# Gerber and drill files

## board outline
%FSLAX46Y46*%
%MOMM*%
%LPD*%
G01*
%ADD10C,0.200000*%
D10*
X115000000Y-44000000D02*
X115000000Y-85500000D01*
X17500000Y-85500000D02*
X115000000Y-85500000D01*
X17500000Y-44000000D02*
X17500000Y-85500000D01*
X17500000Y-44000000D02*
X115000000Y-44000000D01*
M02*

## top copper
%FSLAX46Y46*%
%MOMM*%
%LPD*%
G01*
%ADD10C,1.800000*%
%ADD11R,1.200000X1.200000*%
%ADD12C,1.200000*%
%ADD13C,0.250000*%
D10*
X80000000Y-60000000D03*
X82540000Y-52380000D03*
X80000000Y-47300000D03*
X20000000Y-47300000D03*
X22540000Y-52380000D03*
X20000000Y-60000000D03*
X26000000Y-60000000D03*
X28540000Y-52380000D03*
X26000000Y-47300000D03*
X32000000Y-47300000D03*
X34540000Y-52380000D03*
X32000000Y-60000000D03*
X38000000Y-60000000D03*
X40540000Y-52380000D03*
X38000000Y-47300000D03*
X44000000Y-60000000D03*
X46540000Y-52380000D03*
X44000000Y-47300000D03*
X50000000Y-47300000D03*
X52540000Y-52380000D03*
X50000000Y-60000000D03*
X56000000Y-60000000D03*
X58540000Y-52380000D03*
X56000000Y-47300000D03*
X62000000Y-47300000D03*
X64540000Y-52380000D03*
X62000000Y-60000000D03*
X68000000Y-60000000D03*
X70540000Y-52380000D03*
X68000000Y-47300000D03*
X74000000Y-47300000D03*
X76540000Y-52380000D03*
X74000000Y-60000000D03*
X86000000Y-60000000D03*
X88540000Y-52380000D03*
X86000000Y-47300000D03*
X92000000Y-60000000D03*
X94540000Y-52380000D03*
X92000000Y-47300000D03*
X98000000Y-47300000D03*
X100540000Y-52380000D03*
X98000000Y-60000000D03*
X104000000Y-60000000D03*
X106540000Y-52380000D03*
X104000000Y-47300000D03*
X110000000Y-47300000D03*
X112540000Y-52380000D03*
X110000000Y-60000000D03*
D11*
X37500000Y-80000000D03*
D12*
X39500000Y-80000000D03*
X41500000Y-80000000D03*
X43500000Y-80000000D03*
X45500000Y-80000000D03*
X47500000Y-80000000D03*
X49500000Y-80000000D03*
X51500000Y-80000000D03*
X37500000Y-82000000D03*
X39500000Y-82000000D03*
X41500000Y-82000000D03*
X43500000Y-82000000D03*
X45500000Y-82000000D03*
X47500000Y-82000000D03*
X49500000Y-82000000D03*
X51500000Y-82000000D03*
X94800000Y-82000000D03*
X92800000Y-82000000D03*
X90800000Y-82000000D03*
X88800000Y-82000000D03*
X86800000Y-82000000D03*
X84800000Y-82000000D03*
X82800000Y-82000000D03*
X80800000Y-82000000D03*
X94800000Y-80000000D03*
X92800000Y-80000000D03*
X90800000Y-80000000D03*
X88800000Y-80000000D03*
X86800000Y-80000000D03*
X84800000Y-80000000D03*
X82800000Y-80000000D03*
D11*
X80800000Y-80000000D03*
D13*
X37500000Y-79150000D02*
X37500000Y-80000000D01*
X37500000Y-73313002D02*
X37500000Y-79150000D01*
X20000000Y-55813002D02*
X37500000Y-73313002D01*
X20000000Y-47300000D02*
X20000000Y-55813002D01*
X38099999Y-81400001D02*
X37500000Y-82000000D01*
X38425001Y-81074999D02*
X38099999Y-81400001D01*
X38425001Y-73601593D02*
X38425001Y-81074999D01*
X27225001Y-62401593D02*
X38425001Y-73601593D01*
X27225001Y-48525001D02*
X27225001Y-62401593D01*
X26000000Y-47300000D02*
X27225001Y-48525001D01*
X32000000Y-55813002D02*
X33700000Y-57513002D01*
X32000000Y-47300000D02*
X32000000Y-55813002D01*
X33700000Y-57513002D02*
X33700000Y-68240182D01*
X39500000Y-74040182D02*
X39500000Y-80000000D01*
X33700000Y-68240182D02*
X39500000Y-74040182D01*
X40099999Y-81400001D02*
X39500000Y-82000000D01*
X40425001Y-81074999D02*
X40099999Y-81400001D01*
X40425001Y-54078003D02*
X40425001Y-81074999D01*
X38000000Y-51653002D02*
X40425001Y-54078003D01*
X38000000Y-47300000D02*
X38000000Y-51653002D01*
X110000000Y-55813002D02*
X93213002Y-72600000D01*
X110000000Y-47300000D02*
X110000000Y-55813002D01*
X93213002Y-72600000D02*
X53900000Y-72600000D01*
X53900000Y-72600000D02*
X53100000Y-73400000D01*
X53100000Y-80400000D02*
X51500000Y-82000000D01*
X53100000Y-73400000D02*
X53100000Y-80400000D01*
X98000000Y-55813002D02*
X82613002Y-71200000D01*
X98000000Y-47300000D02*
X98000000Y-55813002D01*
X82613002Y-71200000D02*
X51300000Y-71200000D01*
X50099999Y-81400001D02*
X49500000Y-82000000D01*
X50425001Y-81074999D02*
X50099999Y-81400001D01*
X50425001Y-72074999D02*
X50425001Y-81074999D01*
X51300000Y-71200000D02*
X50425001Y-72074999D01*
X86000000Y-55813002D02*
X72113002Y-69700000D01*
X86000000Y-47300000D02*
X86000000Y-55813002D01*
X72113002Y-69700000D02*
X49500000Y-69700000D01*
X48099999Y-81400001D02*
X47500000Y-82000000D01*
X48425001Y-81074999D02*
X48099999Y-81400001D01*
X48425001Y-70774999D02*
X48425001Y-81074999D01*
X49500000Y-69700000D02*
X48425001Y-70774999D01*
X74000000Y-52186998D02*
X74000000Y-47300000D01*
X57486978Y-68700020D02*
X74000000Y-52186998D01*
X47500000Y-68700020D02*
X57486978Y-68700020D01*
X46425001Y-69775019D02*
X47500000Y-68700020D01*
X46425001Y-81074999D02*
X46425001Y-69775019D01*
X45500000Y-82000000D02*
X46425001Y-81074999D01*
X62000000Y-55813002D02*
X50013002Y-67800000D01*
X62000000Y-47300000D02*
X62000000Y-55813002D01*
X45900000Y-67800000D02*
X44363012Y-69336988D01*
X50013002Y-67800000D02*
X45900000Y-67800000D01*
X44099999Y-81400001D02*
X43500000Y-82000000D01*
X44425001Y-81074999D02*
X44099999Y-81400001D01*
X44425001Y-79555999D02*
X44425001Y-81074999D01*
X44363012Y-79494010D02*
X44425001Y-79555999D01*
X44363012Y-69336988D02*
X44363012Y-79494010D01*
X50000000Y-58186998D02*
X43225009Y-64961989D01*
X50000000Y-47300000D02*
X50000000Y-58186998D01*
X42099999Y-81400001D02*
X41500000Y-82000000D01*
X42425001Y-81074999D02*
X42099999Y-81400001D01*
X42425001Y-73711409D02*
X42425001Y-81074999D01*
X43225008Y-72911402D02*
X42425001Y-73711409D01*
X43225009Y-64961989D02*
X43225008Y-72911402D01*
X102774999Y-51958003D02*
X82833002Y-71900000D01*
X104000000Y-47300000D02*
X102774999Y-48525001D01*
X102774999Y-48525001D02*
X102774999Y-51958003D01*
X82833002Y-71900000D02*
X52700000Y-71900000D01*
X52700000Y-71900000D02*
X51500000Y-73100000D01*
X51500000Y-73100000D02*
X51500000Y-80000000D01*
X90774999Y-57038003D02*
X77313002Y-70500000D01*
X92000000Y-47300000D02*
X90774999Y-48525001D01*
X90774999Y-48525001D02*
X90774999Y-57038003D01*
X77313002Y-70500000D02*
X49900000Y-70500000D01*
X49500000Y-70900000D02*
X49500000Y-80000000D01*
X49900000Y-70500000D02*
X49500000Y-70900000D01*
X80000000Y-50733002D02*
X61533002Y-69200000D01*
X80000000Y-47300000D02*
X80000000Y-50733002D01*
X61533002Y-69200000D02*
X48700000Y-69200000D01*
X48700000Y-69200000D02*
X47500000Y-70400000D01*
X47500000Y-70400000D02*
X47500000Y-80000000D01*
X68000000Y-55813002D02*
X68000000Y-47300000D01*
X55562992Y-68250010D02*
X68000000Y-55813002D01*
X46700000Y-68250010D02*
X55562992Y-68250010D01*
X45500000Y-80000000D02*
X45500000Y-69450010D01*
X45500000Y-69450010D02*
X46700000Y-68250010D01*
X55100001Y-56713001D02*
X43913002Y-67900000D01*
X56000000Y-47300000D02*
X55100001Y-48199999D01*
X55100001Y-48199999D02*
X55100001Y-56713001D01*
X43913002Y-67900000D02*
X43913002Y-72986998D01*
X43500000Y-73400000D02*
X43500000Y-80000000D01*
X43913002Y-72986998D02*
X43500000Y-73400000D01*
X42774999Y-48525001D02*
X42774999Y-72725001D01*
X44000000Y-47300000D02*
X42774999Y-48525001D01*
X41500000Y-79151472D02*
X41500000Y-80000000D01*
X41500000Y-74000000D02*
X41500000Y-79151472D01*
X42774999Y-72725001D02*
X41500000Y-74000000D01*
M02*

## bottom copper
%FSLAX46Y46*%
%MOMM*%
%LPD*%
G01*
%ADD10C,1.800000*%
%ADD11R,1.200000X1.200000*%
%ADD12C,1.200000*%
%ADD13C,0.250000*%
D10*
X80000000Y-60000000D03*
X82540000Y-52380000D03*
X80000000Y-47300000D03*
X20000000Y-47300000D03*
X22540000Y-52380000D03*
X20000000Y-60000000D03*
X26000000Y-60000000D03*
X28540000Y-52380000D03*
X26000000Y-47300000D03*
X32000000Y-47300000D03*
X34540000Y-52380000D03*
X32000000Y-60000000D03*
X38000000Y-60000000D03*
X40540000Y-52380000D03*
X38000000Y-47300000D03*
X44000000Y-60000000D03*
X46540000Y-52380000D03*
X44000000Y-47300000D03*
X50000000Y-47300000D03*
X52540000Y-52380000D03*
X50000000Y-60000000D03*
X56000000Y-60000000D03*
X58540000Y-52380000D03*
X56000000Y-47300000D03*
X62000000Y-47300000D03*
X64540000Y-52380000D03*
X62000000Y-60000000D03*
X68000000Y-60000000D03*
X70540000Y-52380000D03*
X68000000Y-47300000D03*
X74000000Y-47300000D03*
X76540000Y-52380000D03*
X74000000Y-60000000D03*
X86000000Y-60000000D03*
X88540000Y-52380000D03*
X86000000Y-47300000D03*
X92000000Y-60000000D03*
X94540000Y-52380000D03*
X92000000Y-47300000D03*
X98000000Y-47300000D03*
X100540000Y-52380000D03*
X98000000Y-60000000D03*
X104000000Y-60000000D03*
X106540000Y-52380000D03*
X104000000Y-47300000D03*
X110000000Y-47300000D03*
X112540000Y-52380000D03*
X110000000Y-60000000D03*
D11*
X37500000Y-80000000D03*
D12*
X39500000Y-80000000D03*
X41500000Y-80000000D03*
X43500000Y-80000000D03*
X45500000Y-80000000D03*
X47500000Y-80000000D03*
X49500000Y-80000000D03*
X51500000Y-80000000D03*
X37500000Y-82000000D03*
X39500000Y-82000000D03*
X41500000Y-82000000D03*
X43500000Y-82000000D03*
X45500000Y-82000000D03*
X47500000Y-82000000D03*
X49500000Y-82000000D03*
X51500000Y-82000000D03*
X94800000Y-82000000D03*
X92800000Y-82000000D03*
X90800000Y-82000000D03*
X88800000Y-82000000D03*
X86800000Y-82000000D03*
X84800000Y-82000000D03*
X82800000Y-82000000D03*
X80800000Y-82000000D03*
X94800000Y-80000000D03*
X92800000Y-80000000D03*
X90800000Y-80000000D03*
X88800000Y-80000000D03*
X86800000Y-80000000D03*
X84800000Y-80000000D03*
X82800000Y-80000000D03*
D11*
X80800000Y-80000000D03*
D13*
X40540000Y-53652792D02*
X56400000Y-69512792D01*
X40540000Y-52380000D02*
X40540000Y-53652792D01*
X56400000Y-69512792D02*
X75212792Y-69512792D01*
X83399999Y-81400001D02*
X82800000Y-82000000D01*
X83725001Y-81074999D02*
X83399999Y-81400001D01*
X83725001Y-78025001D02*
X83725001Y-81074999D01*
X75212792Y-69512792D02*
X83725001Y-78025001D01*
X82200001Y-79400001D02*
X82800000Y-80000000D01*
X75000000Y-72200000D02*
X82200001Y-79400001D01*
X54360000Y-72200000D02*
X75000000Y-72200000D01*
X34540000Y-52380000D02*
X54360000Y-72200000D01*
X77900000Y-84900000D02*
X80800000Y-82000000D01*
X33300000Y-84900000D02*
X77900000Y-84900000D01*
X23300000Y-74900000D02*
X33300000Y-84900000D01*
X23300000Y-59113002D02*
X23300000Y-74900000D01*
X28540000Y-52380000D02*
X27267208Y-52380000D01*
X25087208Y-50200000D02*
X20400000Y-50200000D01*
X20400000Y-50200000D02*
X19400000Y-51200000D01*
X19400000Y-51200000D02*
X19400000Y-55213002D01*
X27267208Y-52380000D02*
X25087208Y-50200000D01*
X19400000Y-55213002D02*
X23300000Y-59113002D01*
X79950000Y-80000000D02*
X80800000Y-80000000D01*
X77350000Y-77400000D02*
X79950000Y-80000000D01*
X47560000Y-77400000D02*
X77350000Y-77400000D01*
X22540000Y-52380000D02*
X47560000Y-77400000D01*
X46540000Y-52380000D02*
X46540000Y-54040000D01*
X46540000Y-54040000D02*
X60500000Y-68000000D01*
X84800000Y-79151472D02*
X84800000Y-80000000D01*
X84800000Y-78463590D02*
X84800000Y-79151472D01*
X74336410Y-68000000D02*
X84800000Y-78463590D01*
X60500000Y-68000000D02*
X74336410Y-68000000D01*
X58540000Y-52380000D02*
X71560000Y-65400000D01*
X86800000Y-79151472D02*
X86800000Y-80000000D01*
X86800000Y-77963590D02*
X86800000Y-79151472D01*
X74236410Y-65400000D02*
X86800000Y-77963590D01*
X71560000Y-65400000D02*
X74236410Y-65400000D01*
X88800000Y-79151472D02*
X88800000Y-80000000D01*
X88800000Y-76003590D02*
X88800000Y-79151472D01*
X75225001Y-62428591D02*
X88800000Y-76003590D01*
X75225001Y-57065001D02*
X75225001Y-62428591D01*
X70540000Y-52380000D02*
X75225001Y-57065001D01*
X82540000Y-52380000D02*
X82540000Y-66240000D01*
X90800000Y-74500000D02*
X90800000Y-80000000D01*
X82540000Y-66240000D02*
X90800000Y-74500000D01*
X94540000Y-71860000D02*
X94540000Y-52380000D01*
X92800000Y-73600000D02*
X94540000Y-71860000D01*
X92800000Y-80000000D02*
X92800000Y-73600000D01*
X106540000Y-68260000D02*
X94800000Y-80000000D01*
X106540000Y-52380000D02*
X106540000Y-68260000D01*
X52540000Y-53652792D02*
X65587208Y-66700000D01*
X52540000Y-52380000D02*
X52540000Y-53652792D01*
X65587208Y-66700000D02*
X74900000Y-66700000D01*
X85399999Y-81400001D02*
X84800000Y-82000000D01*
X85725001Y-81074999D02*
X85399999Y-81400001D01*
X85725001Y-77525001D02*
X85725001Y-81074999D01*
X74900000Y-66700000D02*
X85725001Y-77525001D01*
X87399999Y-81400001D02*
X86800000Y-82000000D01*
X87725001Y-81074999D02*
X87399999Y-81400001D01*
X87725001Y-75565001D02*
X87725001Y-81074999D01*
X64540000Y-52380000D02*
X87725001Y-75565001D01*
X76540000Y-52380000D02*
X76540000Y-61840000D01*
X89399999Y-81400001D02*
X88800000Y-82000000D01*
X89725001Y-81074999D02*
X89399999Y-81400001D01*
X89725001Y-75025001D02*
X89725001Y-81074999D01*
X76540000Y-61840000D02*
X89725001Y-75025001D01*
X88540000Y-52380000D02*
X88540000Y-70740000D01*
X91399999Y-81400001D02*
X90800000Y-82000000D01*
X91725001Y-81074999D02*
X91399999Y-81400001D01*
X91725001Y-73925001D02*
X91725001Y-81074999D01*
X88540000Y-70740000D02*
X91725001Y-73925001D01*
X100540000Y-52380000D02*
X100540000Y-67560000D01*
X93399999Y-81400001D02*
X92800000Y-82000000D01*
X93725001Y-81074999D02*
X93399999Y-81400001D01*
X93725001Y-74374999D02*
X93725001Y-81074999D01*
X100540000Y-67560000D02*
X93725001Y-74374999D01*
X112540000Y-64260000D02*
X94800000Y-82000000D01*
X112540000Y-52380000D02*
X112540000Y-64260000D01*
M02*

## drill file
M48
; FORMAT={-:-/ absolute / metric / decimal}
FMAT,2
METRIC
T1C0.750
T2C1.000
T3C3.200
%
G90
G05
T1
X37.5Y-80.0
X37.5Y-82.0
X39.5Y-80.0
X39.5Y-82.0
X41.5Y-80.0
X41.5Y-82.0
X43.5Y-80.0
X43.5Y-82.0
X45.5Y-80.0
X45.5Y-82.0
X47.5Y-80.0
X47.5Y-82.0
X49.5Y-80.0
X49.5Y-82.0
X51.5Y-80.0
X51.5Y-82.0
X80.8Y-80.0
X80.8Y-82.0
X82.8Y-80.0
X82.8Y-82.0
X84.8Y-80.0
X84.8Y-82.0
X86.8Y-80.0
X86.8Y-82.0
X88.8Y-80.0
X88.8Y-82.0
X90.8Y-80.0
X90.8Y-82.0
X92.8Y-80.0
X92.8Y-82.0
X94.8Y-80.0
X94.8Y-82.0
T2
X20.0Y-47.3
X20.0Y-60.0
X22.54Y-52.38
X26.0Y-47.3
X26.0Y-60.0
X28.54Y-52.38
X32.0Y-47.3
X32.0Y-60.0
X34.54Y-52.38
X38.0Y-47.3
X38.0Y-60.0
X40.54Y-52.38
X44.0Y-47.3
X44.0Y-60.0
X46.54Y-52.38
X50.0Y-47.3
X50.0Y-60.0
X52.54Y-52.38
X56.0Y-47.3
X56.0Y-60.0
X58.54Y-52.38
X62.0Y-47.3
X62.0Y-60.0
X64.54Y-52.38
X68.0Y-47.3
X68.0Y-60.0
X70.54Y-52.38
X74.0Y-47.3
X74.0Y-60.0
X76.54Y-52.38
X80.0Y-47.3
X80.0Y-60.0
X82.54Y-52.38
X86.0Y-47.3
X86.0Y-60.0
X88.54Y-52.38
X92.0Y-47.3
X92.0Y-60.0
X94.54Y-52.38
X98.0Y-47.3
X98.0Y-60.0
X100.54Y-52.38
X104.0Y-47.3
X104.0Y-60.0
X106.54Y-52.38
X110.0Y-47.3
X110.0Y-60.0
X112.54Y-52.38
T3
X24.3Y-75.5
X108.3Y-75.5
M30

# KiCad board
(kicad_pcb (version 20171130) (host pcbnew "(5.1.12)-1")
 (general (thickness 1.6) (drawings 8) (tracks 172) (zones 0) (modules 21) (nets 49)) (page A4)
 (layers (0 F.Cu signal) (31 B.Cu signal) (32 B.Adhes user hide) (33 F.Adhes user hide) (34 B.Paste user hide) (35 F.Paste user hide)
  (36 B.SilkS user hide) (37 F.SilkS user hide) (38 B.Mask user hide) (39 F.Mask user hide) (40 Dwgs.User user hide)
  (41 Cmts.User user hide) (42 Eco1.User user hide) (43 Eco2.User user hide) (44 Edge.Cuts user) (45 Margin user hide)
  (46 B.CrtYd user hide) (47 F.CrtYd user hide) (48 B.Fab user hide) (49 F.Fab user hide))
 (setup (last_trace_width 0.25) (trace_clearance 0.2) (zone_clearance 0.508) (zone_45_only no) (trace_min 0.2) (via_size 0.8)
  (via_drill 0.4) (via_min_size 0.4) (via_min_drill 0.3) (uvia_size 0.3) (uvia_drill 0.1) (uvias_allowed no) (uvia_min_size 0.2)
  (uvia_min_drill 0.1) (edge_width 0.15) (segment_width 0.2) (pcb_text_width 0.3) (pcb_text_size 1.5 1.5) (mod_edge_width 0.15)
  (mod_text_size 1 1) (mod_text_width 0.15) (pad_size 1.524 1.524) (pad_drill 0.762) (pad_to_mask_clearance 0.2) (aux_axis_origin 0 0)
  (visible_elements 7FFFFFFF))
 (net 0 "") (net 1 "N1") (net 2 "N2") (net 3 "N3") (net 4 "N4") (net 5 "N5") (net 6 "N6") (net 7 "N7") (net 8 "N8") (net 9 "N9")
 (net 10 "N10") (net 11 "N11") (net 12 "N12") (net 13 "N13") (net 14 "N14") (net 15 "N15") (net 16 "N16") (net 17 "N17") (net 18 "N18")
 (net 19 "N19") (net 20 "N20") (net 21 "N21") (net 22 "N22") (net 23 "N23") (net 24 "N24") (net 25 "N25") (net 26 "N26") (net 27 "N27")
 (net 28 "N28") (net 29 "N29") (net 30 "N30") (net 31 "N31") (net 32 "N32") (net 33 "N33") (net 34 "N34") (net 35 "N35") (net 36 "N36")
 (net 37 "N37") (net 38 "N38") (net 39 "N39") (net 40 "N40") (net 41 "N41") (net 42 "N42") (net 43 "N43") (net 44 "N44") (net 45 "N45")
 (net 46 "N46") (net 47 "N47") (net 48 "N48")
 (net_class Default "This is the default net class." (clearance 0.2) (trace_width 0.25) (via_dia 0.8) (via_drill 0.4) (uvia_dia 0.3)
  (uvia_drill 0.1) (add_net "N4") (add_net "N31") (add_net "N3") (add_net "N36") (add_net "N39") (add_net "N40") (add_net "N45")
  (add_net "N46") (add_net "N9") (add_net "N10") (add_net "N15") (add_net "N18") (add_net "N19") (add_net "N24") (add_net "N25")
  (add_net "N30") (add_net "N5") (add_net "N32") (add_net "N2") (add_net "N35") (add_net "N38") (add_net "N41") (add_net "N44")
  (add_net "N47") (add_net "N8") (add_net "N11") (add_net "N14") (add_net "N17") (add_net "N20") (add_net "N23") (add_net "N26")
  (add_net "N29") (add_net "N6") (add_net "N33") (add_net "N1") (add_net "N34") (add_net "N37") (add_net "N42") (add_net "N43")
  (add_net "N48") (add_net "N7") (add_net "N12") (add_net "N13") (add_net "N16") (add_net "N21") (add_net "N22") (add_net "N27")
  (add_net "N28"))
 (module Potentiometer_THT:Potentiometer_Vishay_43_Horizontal (layer F.Cu) (at 80 60 270)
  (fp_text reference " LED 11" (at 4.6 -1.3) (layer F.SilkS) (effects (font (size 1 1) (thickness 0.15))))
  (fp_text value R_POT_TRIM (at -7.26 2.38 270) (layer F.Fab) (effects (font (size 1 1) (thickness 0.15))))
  (pad 1 thru_hole circle (at 0 0 270) (size 1.8 1.8) (drill 1) (layers *.Cu *.Mask) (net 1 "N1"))
  (pad 2 thru_hole circle (at -7.62 -2.54 270) (size 1.8 1.8) (drill 1) (layers *.Cu *.Mask) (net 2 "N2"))
  (pad 3 thru_hole circle (at -12.7 0 270) (size 1.8 1.8) (drill 1) (layers *.Cu *.Mask) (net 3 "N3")))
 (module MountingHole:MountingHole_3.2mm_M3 (layer F.Cu) (at 108.3 75.5)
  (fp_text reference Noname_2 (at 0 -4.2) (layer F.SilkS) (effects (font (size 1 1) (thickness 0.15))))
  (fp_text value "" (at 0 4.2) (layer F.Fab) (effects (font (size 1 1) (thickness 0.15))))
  (pad 1 np_thru_hole circle (at 0 0) (size 3.2 3.2) (drill 3.2) (layers *.Cu *.Mask)))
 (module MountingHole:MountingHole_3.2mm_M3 (layer F.Cu) (at 24.3 75.5)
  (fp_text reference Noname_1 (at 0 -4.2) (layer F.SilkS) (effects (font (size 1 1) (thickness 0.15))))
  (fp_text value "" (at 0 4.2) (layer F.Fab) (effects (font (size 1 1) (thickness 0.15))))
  (pad 1 np_thru_hole circle (at 0 0) (size 3.2 3.2) (drill 3.2) (layers *.Cu *.Mask)))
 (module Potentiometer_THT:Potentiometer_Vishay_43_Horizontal (layer F.Cu) (at 20 60 270)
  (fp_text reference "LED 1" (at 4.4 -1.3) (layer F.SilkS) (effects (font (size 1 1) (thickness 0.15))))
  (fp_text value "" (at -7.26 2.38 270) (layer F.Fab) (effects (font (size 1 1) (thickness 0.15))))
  (pad 3 thru_hole circle (at -12.7 0 270) (size 1.8 1.8) (drill 1) (layers *.Cu *.Mask) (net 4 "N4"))
  (pad 2 thru_hole circle (at -7.62 -2.54 270) (size 1.8 1.8) (drill 1) (layers *.Cu *.Mask) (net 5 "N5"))
  (pad 1 thru_hole circle (at 0 0 270) (size 1.8 1.8) (drill 1) (layers *.Cu *.Mask) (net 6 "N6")))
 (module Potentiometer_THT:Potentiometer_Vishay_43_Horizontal (layer F.Cu) (at 26 60 270)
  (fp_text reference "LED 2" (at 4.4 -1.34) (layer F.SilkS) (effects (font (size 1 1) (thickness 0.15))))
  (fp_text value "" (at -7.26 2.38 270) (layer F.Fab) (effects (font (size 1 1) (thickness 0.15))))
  (pad 1 thru_hole circle (at 0 0 270) (size 1.8 1.8) (drill 1) (layers *.Cu *.Mask) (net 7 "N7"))
  (pad 2 thru_hole circle (at -7.62 -2.54 270) (size 1.8 1.8) (drill 1) (layers *.Cu *.Mask) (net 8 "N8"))
  (pad 3 thru_hole circle (at -12.7 0 270) (size 1.8 1.8) (drill 1) (layers *.Cu *.Mask) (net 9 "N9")))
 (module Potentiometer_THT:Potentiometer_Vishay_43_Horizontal (layer F.Cu) (at 32 60 270)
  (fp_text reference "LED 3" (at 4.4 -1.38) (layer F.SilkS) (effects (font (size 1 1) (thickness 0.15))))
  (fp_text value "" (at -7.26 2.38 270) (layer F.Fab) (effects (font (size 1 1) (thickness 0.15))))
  (pad 3 thru_hole circle (at -12.7 0 270) (size 1.8 1.8) (drill 1) (layers *.Cu *.Mask) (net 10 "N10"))
  (pad 2 thru_hole circle (at -7.62 -2.54 270) (size 1.8 1.8) (drill 1) (layers *.Cu *.Mask) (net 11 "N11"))
  (pad 1 thru_hole circle (at 0 0 270) (size 1.8 1.8) (drill 1) (layers *.Cu *.Mask) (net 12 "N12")))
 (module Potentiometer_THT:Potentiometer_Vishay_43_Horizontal (layer F.Cu) (at 38 60 270)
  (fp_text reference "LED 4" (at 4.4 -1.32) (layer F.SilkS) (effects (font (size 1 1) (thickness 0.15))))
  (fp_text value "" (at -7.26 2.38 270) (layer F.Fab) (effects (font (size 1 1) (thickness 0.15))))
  (pad 1 thru_hole circle (at 0 0 270) (size 1.8 1.8) (drill 1) (layers *.Cu *.Mask) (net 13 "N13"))
  (pad 2 thru_hole circle (at -7.62 -2.54 270) (size 1.8 1.8) (drill 1) (layers *.Cu *.Mask) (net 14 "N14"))
  (pad 3 thru_hole circle (at -12.7 0 270) (size 1.8 1.8) (drill 1) (layers *.Cu *.Mask) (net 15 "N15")))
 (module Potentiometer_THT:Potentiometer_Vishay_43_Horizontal (layer F.Cu) (at 44 60 270)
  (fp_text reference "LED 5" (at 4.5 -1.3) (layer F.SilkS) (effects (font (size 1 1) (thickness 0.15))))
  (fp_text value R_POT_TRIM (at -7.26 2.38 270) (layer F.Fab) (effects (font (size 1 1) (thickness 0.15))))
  (pad 1 thru_hole circle (at 0 0 270) (size 1.8 1.8) (drill 1) (layers *.Cu *.Mask) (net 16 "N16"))
  (pad 2 thru_hole circle (at -7.62 -2.54 270) (size 1.8 1.8) (drill 1) (layers *.Cu *.Mask) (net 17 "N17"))
  (pad 3 thru_hole circle (at -12.7 0 270) (size 1.8 1.8) (drill 1) (layers *.Cu *.Mask) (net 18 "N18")))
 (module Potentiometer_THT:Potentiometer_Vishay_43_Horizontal (layer F.Cu) (at 50 60 270)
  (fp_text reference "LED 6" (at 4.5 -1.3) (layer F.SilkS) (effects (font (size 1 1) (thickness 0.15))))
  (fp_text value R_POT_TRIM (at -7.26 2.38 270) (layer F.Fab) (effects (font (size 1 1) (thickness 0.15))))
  (pad 3 thru_hole circle (at -12.7 0 270) (size 1.8 1.8) (drill 1) (layers *.Cu *.Mask) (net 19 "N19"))
  (pad 2 thru_hole circle (at -7.62 -2.54 270) (size 1.8 1.8) (drill 1) (layers *.Cu *.Mask) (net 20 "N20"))
  (pad 1 thru_hole circle (at 0 0 270) (size 1.8 1.8) (drill 1) (layers *.Cu *.Mask) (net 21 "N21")))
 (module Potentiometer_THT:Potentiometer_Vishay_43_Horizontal (layer F.Cu) (at 56 60 270)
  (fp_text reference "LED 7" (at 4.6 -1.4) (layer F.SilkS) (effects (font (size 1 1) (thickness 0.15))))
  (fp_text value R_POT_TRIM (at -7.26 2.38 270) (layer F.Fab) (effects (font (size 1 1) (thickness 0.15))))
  (pad 1 thru_hole circle (at 0 0 270) (size 1.8 1.8) (drill 1) (layers *.Cu *.Mask) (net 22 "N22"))
  (pad 2 thru_hole circle (at -7.62 -2.54 270) (size 1.8 1.8) (drill 1) (layers *.Cu *.Mask) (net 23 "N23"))
  (pad 3 thru_hole circle (at -12.7 0 270) (size 1.8 1.8) (drill 1) (layers *.Cu *.Mask) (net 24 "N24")))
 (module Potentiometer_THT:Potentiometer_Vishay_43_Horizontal (layer F.Cu) (at 62 60 270)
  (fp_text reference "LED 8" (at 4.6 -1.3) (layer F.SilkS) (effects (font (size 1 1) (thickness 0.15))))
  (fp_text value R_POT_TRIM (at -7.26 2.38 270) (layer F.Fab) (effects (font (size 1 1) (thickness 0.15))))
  (pad 3 thru_hole circle (at -12.7 0 270) (size 1.8 1.8) (drill 1) (layers *.Cu *.Mask) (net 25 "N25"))
  (pad 2 thru_hole circle (at -7.62 -2.54 270) (size 1.8 1.8) (drill 1) (layers *.Cu *.Mask) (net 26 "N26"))
  (pad 1 thru_hole circle (at 0 0 270) (size 1.8 1.8) (drill 1) (layers *.Cu *.Mask) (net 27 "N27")))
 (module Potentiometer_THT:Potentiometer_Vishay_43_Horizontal (layer F.Cu) (at 68 60 270)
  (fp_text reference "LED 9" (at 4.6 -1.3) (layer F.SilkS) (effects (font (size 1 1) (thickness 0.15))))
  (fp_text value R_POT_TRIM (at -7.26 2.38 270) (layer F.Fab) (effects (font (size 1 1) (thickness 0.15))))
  (pad 1 thru_hole circle (at 0 0 270) (size 1.8 1.8) (drill 1) (layers *.Cu *.Mask) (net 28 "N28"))
  (pad 2 thru_hole circle (at -7.62 -2.54 270) (size 1.8 1.8) (drill 1) (layers *.Cu *.Mask) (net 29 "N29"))
  (pad 3 thru_hole circle (at -12.7 0 270) (size 1.8 1.8) (drill 1) (layers *.Cu *.Mask) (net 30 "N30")))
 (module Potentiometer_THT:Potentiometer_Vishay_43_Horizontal (layer F.Cu) (at 74 60 270)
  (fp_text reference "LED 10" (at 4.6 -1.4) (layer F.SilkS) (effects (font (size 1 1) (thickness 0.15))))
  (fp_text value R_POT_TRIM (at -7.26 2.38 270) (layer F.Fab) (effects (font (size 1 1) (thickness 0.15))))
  (pad 3 thru_hole circle (at -12.7 0 270) (size 1.8 1.8) (drill 1) (layers *.Cu *.Mask) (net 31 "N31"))
  (pad 2 thru_hole circle (at -7.62 -2.54 270) (size 1.8 1.8) (drill 1) (layers *.Cu *.Mask) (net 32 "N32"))
  (pad 1 thru_hole circle (at 0 0 270) (size 1.8 1.8) (drill 1) (layers *.Cu *.Mask) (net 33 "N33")))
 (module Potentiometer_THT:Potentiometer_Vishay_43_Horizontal (layer F.Cu) (at 86 60 270)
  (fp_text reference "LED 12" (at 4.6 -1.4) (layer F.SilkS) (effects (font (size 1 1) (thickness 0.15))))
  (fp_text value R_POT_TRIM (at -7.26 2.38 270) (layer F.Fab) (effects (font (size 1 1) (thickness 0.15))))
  (pad 1 thru_hole circle (at 0 0 270) (size 1.8 1.8) (drill 1) (layers *.Cu *.Mask) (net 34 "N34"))
  (pad 2 thru_hole circle (at -7.62 -2.54 270) (size 1.8 1.8) (drill 1) (layers *.Cu *.Mask) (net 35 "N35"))
  (pad 3 thru_hole circle (at -12.7 0 270) (size 1.8 1.8) (drill 1) (layers *.Cu *.Mask) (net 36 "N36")))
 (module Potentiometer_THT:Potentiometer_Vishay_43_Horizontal (layer F.Cu) (at 92 60 270)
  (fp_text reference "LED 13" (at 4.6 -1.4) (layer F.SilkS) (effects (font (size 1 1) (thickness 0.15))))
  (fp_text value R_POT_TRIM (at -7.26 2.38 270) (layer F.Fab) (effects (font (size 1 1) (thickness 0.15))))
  (pad 1 thru_hole circle (at 0 0 270) (size 1.8 1.8) (drill 1) (layers *.Cu *.Mask) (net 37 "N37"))
  (pad 2 thru_hole circle (at -7.62 -2.54 270) (size 1.8 1.8) (drill 1) (layers *.Cu *.Mask) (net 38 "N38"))
  (pad 3 thru_hole circle (at -12.7 0 270) (size 1.8 1.8) (drill 1) (layers *.Cu *.Mask) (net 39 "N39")))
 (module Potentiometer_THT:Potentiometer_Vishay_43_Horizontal (layer F.Cu) (at 98 60 270)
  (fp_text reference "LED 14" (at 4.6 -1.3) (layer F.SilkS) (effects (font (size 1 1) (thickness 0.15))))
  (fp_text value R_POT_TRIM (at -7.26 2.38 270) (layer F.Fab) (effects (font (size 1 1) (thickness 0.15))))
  (pad 3 thru_hole circle (at -12.7 0 270) (size 1.8 1.8) (drill 1) (layers *.Cu *.Mask) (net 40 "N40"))
  (pad 2 thru_hole circle (at -7.62 -2.54 270) (size 1.8 1.8) (drill 1) (layers *.Cu *.Mask) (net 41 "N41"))
  (pad 1 thru_hole circle (at 0 0 270) (size 1.8 1.8) (drill 1) (layers *.Cu *.Mask) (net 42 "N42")))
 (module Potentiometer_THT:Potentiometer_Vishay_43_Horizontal (layer F.Cu) (at 104 60 270)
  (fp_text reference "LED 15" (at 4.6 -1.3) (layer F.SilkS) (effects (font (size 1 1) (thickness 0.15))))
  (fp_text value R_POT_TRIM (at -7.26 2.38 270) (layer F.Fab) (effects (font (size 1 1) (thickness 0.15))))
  (pad 1 thru_hole circle (at 0 0 270) (size 1.8 1.8) (drill 1) (layers *.Cu *.Mask) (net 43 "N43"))
  (pad 2 thru_hole circle (at -7.62 -2.54 270) (size 1.8 1.8) (drill 1) (layers *.Cu *.Mask) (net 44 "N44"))
  (pad 3 thru_hole circle (at -12.7 0 270) (size 1.8 1.8) (drill 1) (layers *.Cu *.Mask) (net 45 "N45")))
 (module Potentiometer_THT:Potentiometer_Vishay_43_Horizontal (layer F.Cu) (at 110 60 270)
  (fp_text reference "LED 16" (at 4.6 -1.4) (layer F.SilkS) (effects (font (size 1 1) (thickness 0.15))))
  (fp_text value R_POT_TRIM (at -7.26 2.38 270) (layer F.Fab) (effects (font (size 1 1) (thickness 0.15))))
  (pad 3 thru_hole circle (at -12.7 0 270) (size 1.8 1.8) (drill 1) (layers *.Cu *.Mask) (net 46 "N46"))
  (pad 2 thru_hole circle (at -7.62 -2.54 270) (size 1.8 1.8) (drill 1) (layers *.Cu *.Mask) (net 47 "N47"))
  (pad 1 thru_hole circle (at 0 0 270) (size 1.8 1.8) (drill 1) (layers *.Cu *.Mask) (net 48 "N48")))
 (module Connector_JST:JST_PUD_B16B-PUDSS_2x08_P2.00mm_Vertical (layer F.Cu) (at 37.5 80)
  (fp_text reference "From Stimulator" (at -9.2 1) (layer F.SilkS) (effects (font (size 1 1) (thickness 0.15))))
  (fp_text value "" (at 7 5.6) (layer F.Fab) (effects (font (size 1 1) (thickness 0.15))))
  (pad 1 thru_hole rect (at 0 0) (size 1.2 1.2) (drill 0.75) (layers *.Cu *.Mask) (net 4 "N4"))
  (pad 3 thru_hole circle (at 2 0) (size 1.2 1.2) (drill 0.75) (layers *.Cu *.Mask) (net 10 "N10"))
  (pad 5 thru_hole circle (at 4 0) (size 1.2 1.2) (drill 0.75) (layers *.Cu *.Mask) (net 18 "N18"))
  (pad 7 thru_hole circle (at 6 0) (size 1.2 1.2) (drill 0.75) (layers *.Cu *.Mask) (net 24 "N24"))
  (pad 9 thru_hole circle (at 8 0) (size 1.2 1.2) (drill 0.75) (layers *.Cu *.Mask) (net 30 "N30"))
  (pad 11 thru_hole circle (at 10 0) (size 1.2 1.2) (drill 0.75) (layers *.Cu *.Mask) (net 3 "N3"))
  (pad 13 thru_hole circle (at 12 0) (size 1.2 1.2) (drill 0.75) (layers *.Cu *.Mask) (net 39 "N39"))
  (pad 15 thru_hole circle (at 14 0) (size 1.2 1.2) (drill 0.75) (layers *.Cu *.Mask) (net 45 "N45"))
  (pad 2 thru_hole circle (at 0 2) (size 1.2 1.2) (drill 0.75) (layers *.Cu *.Mask) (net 9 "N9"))
  (pad 4 thru_hole circle (at 2 2) (size 1.2 1.2) (drill 0.75) (layers *.Cu *.Mask) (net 15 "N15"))
  (pad 6 thru_hole circle (at 4 2) (size 1.2 1.2) (drill 0.75) (layers *.Cu *.Mask) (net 19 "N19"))
  (pad 8 thru_hole circle (at 6 2) (size 1.2 1.2) (drill 0.75) (layers *.Cu *.Mask) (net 25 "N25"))
  (pad 10 thru_hole circle (at 8 2) (size 1.2 1.2) (drill 0.75) (layers *.Cu *.Mask) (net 31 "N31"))
  (pad 12 thru_hole circle (at 10 2) (size 1.2 1.2) (drill 0.75) (layers *.Cu *.Mask) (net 36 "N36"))
  (pad 14 thru_hole circle (at 12 2) (size 1.2 1.2) (drill 0.75) (layers *.Cu *.Mask) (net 40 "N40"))
  (pad 16 thru_hole circle (at 14 2) (size 1.2 1.2) (drill 0.75) (layers *.Cu *.Mask) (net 46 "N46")))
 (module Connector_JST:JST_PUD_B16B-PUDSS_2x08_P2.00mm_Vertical (layer F.Cu) (at 80.8 80)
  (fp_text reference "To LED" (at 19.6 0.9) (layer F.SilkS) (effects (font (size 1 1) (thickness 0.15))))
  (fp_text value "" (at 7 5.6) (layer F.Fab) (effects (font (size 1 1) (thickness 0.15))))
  (pad 16 thru_hole circle (at 14 2) (size 1.2 1.2) (drill 0.75) (layers *.Cu *.Mask) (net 47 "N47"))
  (pad 14 thru_hole circle (at 12 2) (size 1.2 1.2) (drill 0.75) (layers *.Cu *.Mask) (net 41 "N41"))
  (pad 12 thru_hole circle (at 10 2) (size 1.2 1.2) (drill 0.75) (layers *.Cu *.Mask) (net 35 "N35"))
  (pad 10 thru_hole circle (at 8 2) (size 1.2 1.2) (drill 0.75) (layers *.Cu *.Mask) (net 32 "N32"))
  (pad 8 thru_hole circle (at 6 2) (size 1.2 1.2) (drill 0.75) (layers *.Cu *.Mask) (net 26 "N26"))
  (pad 6 thru_hole circle (at 4 2) (size 1.2 1.2) (drill 0.75) (layers *.Cu *.Mask) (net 20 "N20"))
  (pad 4 thru_hole circle (at 2 2) (size 1.2 1.2) (drill 0.75) (layers *.Cu *.Mask) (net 14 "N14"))
  (pad 2 thru_hole circle (at 0 2) (size 1.2 1.2) (drill 0.75) (layers *.Cu *.Mask) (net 8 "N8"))
  (pad 15 thru_hole circle (at 14 0) (size 1.2 1.2) (drill 0.75) (layers *.Cu *.Mask) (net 44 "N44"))
  (pad 13 thru_hole circle (at 12 0) (size 1.2 1.2) (drill 0.75) (layers *.Cu *.Mask) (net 38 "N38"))
  (pad 11 thru_hole circle (at 10 0) (size 1.2 1.2) (drill 0.75) (layers *.Cu *.Mask) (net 2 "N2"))
  (pad 9 thru_hole circle (at 8 0) (size 1.2 1.2) (drill 0.75) (layers *.Cu *.Mask) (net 29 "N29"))
  (pad 7 thru_hole circle (at 6 0) (size 1.2 1.2) (drill 0.75) (layers *.Cu *.Mask) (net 23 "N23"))
  (pad 5 thru_hole circle (at 4 0) (size 1.2 1.2) (drill 0.75) (layers *.Cu *.Mask) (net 17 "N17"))
  (pad 3 thru_hole circle (at 2 0) (size 1.2 1.2) (drill 0.75) (layers *.Cu *.Mask) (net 11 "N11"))
  (pad 1 thru_hole rect (at 0 0) (size 1.2 1.2) (drill 0.75) (layers *.Cu *.Mask) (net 5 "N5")))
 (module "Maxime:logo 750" (layer F.Cu) (at 67.8 80.4)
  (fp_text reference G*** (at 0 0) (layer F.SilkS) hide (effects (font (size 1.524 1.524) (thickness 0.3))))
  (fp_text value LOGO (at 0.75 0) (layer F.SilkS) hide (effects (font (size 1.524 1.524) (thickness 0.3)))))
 (gr_line (start 115 44) (end 115 85.5) (layer Edge.Cuts) (width 0.2))
 (gr_line (start 17.5 85.5) (end 115 85.5) (layer Edge.Cuts) (width 0.2))
 (gr_line (start 17.5 44) (end 17.5 85.5) (layer Edge.Cuts) (width 0.2))
 (gr_line (start 17.5 44) (end 115 44) (layer Edge.Cuts) (width 0.2))
 (segment (start 37.5 79.15) (end 37.5 80) (width 0.25) (layer F.Cu) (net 4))
 (segment (start 37.5 73.313002) (end 37.5 79.15) (width 0.25) (layer F.Cu) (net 4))
 (segment (start 20 55.813002) (end 37.5 73.313002) (width 0.25) (layer F.Cu) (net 4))
 (segment (start 20 47.3) (end 20 55.813002) (width 0.25) (layer F.Cu) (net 4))
 (segment (start 38.099999 81.400001) (end 37.5 82) (width 0.25) (layer F.Cu) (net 9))
 (segment (start 38.425001 81.074999) (end 38.099999 81.400001) (width 0.25) (layer F.Cu) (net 9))
 (segment (start 38.425001 73.601593) (end 38.425001 81.074999) (width 0.25) (layer F.Cu) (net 9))
 (segment (start 27.225001 62.401593) (end 38.425001 73.601593) (width 0.25) (layer F.Cu) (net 9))
 (segment (start 27.225001 48.525001) (end 27.225001 62.401593) (width 0.25) (layer F.Cu) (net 9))
 (segment (start 26 47.3) (end 27.225001 48.525001) (width 0.25) (layer F.Cu) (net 9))
 (segment (start 32 55.813002) (end 33.7 57.513002) (width 0.25) (layer F.Cu) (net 10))
 (segment (start 32 47.3) (end 32 55.813002) (width 0.25) (layer F.Cu) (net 10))
 (segment (start 33.7 57.513002) (end 33.7 68.240182) (width 0.25) (layer F.Cu) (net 10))
 (segment (start 39.5 74.040182) (end 39.5 80) (width 0.25) (layer F.Cu) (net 10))
 (segment (start 33.7 68.240182) (end 39.5 74.040182) (width 0.25) (layer F.Cu) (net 10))
 (segment (start 40.099999 81.400001) (end 39.5 82) (width 0.25) (layer F.Cu) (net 15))
 (segment (start 40.425001 81.074999) (end 40.099999 81.400001) (width 0.25) (layer F.Cu) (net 15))
 (segment (start 40.425001 54.078003) (end 40.425001 81.074999) (width 0.25) (layer F.Cu) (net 15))
 (segment (start 38 51.653002) (end 40.425001 54.078003) (width 0.25) (layer F.Cu) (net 15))
 (segment (start 38 47.3) (end 38 51.653002) (width 0.25) (layer F.Cu) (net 15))
 (segment (start 40.54 53.652792) (end 56.4 69.512792) (width 0.25) (layer B.Cu) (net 14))
 (segment (start 40.54 52.38) (end 40.54 53.652792) (width 0.25) (layer B.Cu) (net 14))
 (segment (start 56.4 69.512792) (end 75.212792 69.512792) (width 0.25) (layer B.Cu) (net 14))
 (segment (start 83.399999 81.400001) (end 82.8 82) (width 0.25) (layer B.Cu) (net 14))
 (segment (start 83.725001 81.074999) (end 83.399999 81.400001) (width 0.25) (layer B.Cu) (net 14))
 (segment (start 83.725001 78.025001) (end 83.725001 81.074999) (width 0.25) (layer B.Cu) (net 14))
 (segment (start 75.212792 69.512792) (end 83.725001 78.025001) (width 0.25) (layer B.Cu) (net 14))
 (segment (start 82.200001 79.400001) (end 82.8 80) (width 0.25) (layer B.Cu) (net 11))
 (segment (start 75 72.2) (end 82.200001 79.400001) (width 0.25) (layer B.Cu) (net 11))
 (segment (start 54.36 72.2) (end 75 72.2) (width 0.25) (layer B.Cu) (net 11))
 (segment (start 34.54 52.38) (end 54.36 72.2) (width 0.25) (layer B.Cu) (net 11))
 (segment (start 77.9 84.9) (end 80.8 82) (width 0.25) (layer B.Cu) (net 8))
 (segment (start 33.3 84.9) (end 77.9 84.9) (width 0.25) (layer B.Cu) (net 8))
 (segment (start 23.3 74.9) (end 33.3 84.9) (width 0.25) (layer B.Cu) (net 8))
 (segment (start 23.3 59.113002) (end 23.3 74.9) (width 0.25) (layer B.Cu) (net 8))
 (segment (start 28.54 52.38) (end 27.267208 52.38) (width 0.25) (layer B.Cu) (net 8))
 (segment (start 25.087208 50.2) (end 20.4 50.2) (width 0.25) (layer B.Cu) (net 8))
 (segment (start 20.4 50.2) (end 19.4 51.2) (width 0.25) (layer B.Cu) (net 8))
 (segment (start 19.4 51.2) (end 19.4 55.213002) (width 0.25) (layer B.Cu) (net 8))
 (segment (start 27.267208 52.38) (end 25.087208 50.2) (width 0.25) (layer B.Cu) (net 8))
 (segment (start 19.4 55.213002) (end 23.3 59.113002) (width 0.25) (layer B.Cu) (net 8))
 (segment (start 79.95 80) (end 80.8 80) (width 0.25) (layer B.Cu) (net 5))
 (segment (start 77.35 77.4) (end 79.95 80) (width 0.25) (layer B.Cu) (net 5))
 (segment (start 47.56 77.4) (end 77.35 77.4) (width 0.25) (layer B.Cu) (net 5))
 (segment (start 22.54 52.38) (end 47.56 77.4) (width 0.25) (layer B.Cu) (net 5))
 (segment (start 110 55.813002) (end 93.213002 72.6) (width 0.25) (layer F.Cu) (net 46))
 (segment (start 110 47.3) (end 110 55.813002) (width 0.25) (layer F.Cu) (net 46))
 (segment (start 93.213002 72.6) (end 53.9 72.6) (width 0.25) (layer F.Cu) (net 46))
 (segment (start 53.9 72.6) (end 53.1 73.4) (width 0.25) (layer F.Cu) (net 46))
 (segment (start 53.1 80.4) (end 51.5 82) (width 0.25) (layer F.Cu) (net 46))
 (segment (start 53.1 73.4) (end 53.1 80.4) (width 0.25) (layer F.Cu) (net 46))
 (segment (start 98 55.813002) (end 82.613002 71.2) (width 0.25) (layer F.Cu) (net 40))
 (segment (start 98 47.3) (end 98 55.813002) (width 0.25) (layer F.Cu) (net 40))
 (segment (start 82.613002 71.2) (end 51.3 71.2) (width 0.25) (layer F.Cu) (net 40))
 (segment (start 50.099999 81.400001) (end 49.5 82) (width 0.25) (layer F.Cu) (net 40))
 (segment (start 50.425001 81.074999) (end 50.099999 81.400001) (width 0.25) (layer F.Cu) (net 40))
 (segment (start 50.425001 72.074999) (end 50.425001 81.074999) (width 0.25) (layer F.Cu) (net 40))
 (segment (start 51.3 71.2) (end 50.425001 72.074999) (width 0.25) (layer F.Cu) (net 40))
 (segment (start 86 55.813002) (end 72.113002 69.7) (width 0.25) (layer F.Cu) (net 36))
 (segment (start 86 47.3) (end 86 55.813002) (width 0.25) (layer F.Cu) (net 36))
 (segment (start 72.113002 69.7) (end 49.5 69.7) (width 0.25) (layer F.Cu) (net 36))
 (segment (start 48.099999 81.400001) (end 47.5 82) (width 0.25) (layer F.Cu) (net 36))
 (segment (start 48.425001 81.074999) (end 48.099999 81.400001) (width 0.25) (layer F.Cu) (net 36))
 (segment (start 48.425001 70.774999) (end 48.425001 81.074999) (width 0.25) (layer F.Cu) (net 36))
 (segment (start 49.5 69.7) (end 48.425001 70.774999) (width 0.25) (layer F.Cu) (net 36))
 (segment (start 74 52.186998) (end 74 47.3) (width 0.25) (layer F.Cu) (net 31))
 (segment (start 57.486978 68.70002) (end 74 52.186998) (width 0.25) (layer F.Cu) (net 31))
 (segment (start 47.5 68.70002) (end 57.486978 68.70002) (width 0.25) (layer F.Cu) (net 31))
 (segment (start 46.425001 69.775019) (end 47.5 68.70002) (width 0.25) (layer F.Cu) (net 31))
 (segment (start 46.425001 81.074999) (end 46.425001 69.775019) (width 0.25) (layer F.Cu) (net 31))
 (segment (start 45.5 82) (end 46.425001 81.074999) (width 0.25) (layer F.Cu) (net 31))
 (segment (start 62 55.813002) (end 50.013002 67.8) (width 0.25) (layer F.Cu) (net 25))
 (segment (start 62 47.3) (end 62 55.813002) (width 0.25) (layer F.Cu) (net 25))
 (segment (start 45.9 67.8) (end 44.363012 69.336988) (width 0.25) (layer F.Cu) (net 25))
 (segment (start 50.013002 67.8) (end 45.9 67.8) (width 0.25) (layer F.Cu) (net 25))
 (segment (start 44.099999 81.400001) (end 43.5 82) (width 0.25) (layer F.Cu) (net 25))
 (segment (start 44.425001 81.074999) (end 44.099999 81.400001) (width 0.25) (layer F.Cu) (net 25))
 (segment (start 44.425001 79.555999) (end 44.425001 81.074999) (width 0.25) (layer F.Cu) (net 25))
 (segment (start 44.363012 79.49401) (end 44.425001 79.555999) (width 0.25) (layer F.Cu) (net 25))
 (segment (start 44.363012 69.336988) (end 44.363012 79.49401) (width 0.25) (layer F.Cu) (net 25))
 (segment (start 50 58.186998) (end 43.225009 64.961989) (width 0.25) (layer F.Cu) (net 19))
 (segment (start 50 47.3) (end 50 58.186998) (width 0.25) (layer F.Cu) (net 19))
 (segment (start 42.099999 81.400001) (end 41.5 82) (width 0.25) (layer F.Cu) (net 19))
 (segment (start 42.425001 81.074999) (end 42.099999 81.400001) (width 0.25) (layer F.Cu) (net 19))
 (segment (start 42.425001 73.711409) (end 42.425001 81.074999) (width 0.25) (layer F.Cu) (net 19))
 (segment (start 43.225008 72.911402) (end 42.425001 73.711409) (width 0.25) (layer F.Cu) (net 19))
 (segment (start 43.225009 64.961989) (end 43.225008 72.911402) (width 0.25) (layer F.Cu) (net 19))
 (segment (start 102.774999 51.958003) (end 82.833002 71.9) (width 0.25) (layer F.Cu) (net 45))
 (segment (start 104 47.3) (end 102.774999 48.525001) (width 0.25) (layer F.Cu) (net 45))
 (segment (start 102.774999 48.525001) (end 102.774999 51.958003) (width 0.25) (layer F.Cu) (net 45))
 (segment (start 82.833002 71.9) (end 52.7 71.9) (width 0.25) (layer F.Cu) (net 45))
 (segment (start 52.7 71.9) (end 51.5 73.1) (width 0.25) (layer F.Cu) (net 45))
 (segment (start 51.5 73.1) (end 51.5 80) (width 0.25) (layer F.Cu) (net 45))
 (segment (start 90.774999 57.038003) (end 77.313002 70.5) (width 0.25) (layer F.Cu) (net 39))
 (segment (start 92 47.3) (end 90.774999 48.525001) (width 0.25) (layer F.Cu) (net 39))
 (segment (start 90.774999 48.525001) (end 90.774999 57.038003) (width 0.25) (layer F.Cu) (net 39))
 (segment (start 77.313002 70.5) (end 49.9 70.5) (width 0.25) (layer F.Cu) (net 39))
 (segment (start 49.5 70.9) (end 49.5 80) (width 0.25) (layer F.Cu) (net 39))
 (segment (start 49.9 70.5) (end 49.5 70.9) (width 0.25) (layer F.Cu) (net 39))
 (segment (start 80 50.733002) (end 61.533002 69.2) (width 0.25) (layer F.Cu) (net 3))
 (segment (start 80 47.3) (end 80 50.733002) (width 0.25) (layer F.Cu) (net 3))
 (segment (start 61.533002 69.2) (end 48.7 69.2) (width 0.25) (layer F.Cu) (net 3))
 (segment (start 48.7 69.2) (end 47.5 70.4) (width 0.25) (layer F.Cu) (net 3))
 (segment (start 47.5 70.4) (end 47.5 80) (width 0.25) (layer F.Cu) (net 3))
 (segment (start 68 55.813002) (end 68 47.3) (width 0.25) (layer F.Cu) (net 30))
 (segment (start 55.562992 68.25001) (end 68 55.813002) (width 0.25) (layer F.Cu) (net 30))
 (segment (start 46.7 68.25001) (end 55.562992 68.25001) (width 0.25) (layer F.Cu) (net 30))
 (segment (start 45.5 80) (end 45.5 69.45001) (width 0.25) (layer F.Cu) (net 30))
 (segment (start 45.5 69.45001) (end 46.7 68.25001) (width 0.25) (layer F.Cu) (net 30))
 (segment (start 55.100001 56.713001) (end 43.913002 67.9) (width 0.25) (layer F.Cu) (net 24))
 (segment (start 56 47.3) (end 55.100001 48.199999) (width 0.25) (layer F.Cu) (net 24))
 (segment (start 55.100001 48.199999) (end 55.100001 56.713001) (width 0.25) (layer F.Cu) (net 24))
 (segment (start 43.913002 67.9) (end 43.913002 72.986998) (width 0.25) (layer F.Cu) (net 24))
 (segment (start 43.5 73.4) (end 43.5 80) (width 0.25) (layer F.Cu) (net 24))
 (segment (start 43.913002 72.986998) (end 43.5 73.4) (width 0.25) (layer F.Cu) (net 24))
 (segment (start 42.774999 48.525001) (end 42.774999 72.725001) (width 0.25) (layer F.Cu) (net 18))
 (segment (start 44 47.3) (end 42.774999 48.525001) (width 0.25) (layer F.Cu) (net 18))
 (segment (start 41.5 79.151472) (end 41.5 80) (width 0.25) (layer F.Cu) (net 18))
 (segment (start 41.5 74) (end 41.5 79.151472) (width 0.25) (layer F.Cu) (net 18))
 (segment (start 42.774999 72.725001) (end 41.5 74) (width 0.25) (layer F.Cu) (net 18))
 (segment (start 46.54 52.38) (end 46.54 54.04) (width 0.25) (layer B.Cu) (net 17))
 (segment (start 46.54 54.04) (end 60.5 68) (width 0.25) (layer B.Cu) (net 17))
 (segment (start 84.8 79.151472) (end 84.8 80) (width 0.25) (layer B.Cu) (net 17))
 (segment (start 84.8 78.46359) (end 84.8 79.151472) (width 0.25) (layer B.Cu) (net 17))
 (segment (start 74.33641 68) (end 84.8 78.46359) (width 0.25) (layer B.Cu) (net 17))
 (segment (start 60.5 68) (end 74.33641 68) (width 0.25) (layer B.Cu) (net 17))
 (segment (start 58.54 52.38) (end 71.56 65.4) (width 0.25) (layer B.Cu) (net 23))
 (segment (start 86.8 79.151472) (end 86.8 80) (width 0.25) (layer B.Cu) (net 23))
 (segment (start 86.8 77.96359) (end 86.8 79.151472) (width 0.25) (layer B.Cu) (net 23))
 (segment (start 74.23641 65.4) (end 86.8 77.96359) (width 0.25) (layer B.Cu) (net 23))
 (segment (start 71.56 65.4) (end 74.23641 65.4) (width 0.25) (layer B.Cu) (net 23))
 (segment (start 88.8 79.151472) (end 88.8 80) (width 0.25) (layer B.Cu) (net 29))
 (segment (start 88.8 76.00359) (end 88.8 79.151472) (width 0.25) (layer B.Cu) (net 29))
 (segment (start 75.225001 62.428591) (end 88.8 76.00359) (width 0.25) (layer B.Cu) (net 29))
 (segment (start 75.225001 57.065001) (end 75.225001 62.428591) (width 0.25) (layer B.Cu) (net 29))
 (segment (start 70.54 52.38) (end 75.225001 57.065001) (width 0.25) (layer B.Cu) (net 29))
 (segment (start 82.54 52.38) (end 82.54 66.24) (width 0.25) (layer B.Cu) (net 2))
 (segment (start 90.8 74.5) (end 90.8 80) (width 0.25) (layer B.Cu) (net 2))
 (segment (start 82.54 66.24) (end 90.8 74.5) (width 0.25) (layer B.Cu) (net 2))
 (segment (start 94.54 71.86) (end 94.54 52.38) (width 0.25) (layer B.Cu) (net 38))
 (segment (start 92.8 73.6) (end 94.54 71.86) (width 0.25) (layer B.Cu) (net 38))
 (segment (start 92.8 80) (end 92.8 73.6) (width 0.25) (layer B.Cu) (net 38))
 (segment (start 106.54 68.26) (end 94.8 80) (width 0.25) (layer B.Cu) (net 44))
 (segment (start 106.54 52.38) (end 106.54 68.26) (width 0.25) (layer B.Cu) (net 44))
 (segment (start 52.54 53.652792) (end 65.587208 66.7) (width 0.25) (layer B.Cu) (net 20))
 (segment (start 52.54 52.38) (end 52.54 53.652792) (width 0.25) (layer B.Cu) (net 20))
 (segment (start 65.587208 66.7) (end 74.9 66.7) (width 0.25) (layer B.Cu) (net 20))
 (segment (start 85.399999 81.400001) (end 84.8 82) (width 0.25) (layer B.Cu) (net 20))
 (segment (start 85.725001 81.074999) (end 85.399999 81.400001) (width 0.25) (layer B.Cu) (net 20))
 (segment (start 85.725001 77.525001) (end 85.725001 81.074999) (width 0.25) (layer B.Cu) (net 20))
 (segment (start 74.9 66.7) (end 85.725001 77.525001) (width 0.25) (layer B.Cu) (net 20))
 (segment (start 87.399999 81.400001) (end 86.8 82) (width 0.25) (layer B.Cu) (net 26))
 (segment (start 87.725001 81.074999) (end 87.399999 81.400001) (width 0.25) (layer B.Cu) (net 26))
 (segment (start 87.725001 75.565001) (end 87.725001 81.074999) (width 0.25) (layer B.Cu) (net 26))
 (segment (start 64.54 52.38) (end 87.725001 75.565001) (width 0.25) (layer B.Cu) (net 26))
 (segment (start 76.54 52.38) (end 76.54 61.84) (width 0.25) (layer B.Cu) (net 32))
 (segment (start 89.399999 81.400001) (end 88.8 82) (width 0.25) (layer B.Cu) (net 32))
 (segment (start 89.725001 81.074999) (end 89.399999 81.400001) (width 0.25) (layer B.Cu) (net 32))
 (segment (start 89.725001 75.025001) (end 89.725001 81.074999) (width 0.25) (layer B.Cu) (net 32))
 (segment (start 76.54 61.84) (end 89.725001 75.025001) (width 0.25) (layer B.Cu) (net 32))
 (segment (start 88.54 52.38) (end 88.54 70.74) (width 0.25) (layer B.Cu) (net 35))
 (segment (start 91.399999 81.400001) (end 90.8 82) (width 0.25) (layer B.Cu) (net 35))
 (segment (start 91.725001 81.074999) (end 91.399999 81.400001) (width 0.25) (layer B.Cu) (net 35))
 (segment (start 91.725001 73.925001) (end 91.725001 81.074999) (width 0.25) (layer B.Cu) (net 35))
 (segment (start 88.54 70.74) (end 91.725001 73.925001) (width 0.25) (layer B.Cu) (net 35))
 (segment (start 100.54 52.38) (end 100.54 67.56) (width 0.25) (layer B.Cu) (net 41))
 (segment (start 93.399999 81.400001) (end 92.8 82) (width 0.25) (layer B.Cu) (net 41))
 (segment (start 93.725001 81.074999) (end 93.399999 81.400001) (width 0.25) (layer B.Cu) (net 41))
 (segment (start 93.725001 74.374999) (end 93.725001 81.074999) (width 0.25) (layer B.Cu) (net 41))
 (segment (start 100.54 67.56) (end 93.725001 74.374999) (width 0.25) (layer B.Cu) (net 41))
 (segment (start 112.54 64.26) (end 94.8 82) (width 0.25) (layer B.Cu) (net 47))
 (segment (start 112.54 52.38) (end 112.54 64.26) (width 0.25) (layer B.Cu) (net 47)))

